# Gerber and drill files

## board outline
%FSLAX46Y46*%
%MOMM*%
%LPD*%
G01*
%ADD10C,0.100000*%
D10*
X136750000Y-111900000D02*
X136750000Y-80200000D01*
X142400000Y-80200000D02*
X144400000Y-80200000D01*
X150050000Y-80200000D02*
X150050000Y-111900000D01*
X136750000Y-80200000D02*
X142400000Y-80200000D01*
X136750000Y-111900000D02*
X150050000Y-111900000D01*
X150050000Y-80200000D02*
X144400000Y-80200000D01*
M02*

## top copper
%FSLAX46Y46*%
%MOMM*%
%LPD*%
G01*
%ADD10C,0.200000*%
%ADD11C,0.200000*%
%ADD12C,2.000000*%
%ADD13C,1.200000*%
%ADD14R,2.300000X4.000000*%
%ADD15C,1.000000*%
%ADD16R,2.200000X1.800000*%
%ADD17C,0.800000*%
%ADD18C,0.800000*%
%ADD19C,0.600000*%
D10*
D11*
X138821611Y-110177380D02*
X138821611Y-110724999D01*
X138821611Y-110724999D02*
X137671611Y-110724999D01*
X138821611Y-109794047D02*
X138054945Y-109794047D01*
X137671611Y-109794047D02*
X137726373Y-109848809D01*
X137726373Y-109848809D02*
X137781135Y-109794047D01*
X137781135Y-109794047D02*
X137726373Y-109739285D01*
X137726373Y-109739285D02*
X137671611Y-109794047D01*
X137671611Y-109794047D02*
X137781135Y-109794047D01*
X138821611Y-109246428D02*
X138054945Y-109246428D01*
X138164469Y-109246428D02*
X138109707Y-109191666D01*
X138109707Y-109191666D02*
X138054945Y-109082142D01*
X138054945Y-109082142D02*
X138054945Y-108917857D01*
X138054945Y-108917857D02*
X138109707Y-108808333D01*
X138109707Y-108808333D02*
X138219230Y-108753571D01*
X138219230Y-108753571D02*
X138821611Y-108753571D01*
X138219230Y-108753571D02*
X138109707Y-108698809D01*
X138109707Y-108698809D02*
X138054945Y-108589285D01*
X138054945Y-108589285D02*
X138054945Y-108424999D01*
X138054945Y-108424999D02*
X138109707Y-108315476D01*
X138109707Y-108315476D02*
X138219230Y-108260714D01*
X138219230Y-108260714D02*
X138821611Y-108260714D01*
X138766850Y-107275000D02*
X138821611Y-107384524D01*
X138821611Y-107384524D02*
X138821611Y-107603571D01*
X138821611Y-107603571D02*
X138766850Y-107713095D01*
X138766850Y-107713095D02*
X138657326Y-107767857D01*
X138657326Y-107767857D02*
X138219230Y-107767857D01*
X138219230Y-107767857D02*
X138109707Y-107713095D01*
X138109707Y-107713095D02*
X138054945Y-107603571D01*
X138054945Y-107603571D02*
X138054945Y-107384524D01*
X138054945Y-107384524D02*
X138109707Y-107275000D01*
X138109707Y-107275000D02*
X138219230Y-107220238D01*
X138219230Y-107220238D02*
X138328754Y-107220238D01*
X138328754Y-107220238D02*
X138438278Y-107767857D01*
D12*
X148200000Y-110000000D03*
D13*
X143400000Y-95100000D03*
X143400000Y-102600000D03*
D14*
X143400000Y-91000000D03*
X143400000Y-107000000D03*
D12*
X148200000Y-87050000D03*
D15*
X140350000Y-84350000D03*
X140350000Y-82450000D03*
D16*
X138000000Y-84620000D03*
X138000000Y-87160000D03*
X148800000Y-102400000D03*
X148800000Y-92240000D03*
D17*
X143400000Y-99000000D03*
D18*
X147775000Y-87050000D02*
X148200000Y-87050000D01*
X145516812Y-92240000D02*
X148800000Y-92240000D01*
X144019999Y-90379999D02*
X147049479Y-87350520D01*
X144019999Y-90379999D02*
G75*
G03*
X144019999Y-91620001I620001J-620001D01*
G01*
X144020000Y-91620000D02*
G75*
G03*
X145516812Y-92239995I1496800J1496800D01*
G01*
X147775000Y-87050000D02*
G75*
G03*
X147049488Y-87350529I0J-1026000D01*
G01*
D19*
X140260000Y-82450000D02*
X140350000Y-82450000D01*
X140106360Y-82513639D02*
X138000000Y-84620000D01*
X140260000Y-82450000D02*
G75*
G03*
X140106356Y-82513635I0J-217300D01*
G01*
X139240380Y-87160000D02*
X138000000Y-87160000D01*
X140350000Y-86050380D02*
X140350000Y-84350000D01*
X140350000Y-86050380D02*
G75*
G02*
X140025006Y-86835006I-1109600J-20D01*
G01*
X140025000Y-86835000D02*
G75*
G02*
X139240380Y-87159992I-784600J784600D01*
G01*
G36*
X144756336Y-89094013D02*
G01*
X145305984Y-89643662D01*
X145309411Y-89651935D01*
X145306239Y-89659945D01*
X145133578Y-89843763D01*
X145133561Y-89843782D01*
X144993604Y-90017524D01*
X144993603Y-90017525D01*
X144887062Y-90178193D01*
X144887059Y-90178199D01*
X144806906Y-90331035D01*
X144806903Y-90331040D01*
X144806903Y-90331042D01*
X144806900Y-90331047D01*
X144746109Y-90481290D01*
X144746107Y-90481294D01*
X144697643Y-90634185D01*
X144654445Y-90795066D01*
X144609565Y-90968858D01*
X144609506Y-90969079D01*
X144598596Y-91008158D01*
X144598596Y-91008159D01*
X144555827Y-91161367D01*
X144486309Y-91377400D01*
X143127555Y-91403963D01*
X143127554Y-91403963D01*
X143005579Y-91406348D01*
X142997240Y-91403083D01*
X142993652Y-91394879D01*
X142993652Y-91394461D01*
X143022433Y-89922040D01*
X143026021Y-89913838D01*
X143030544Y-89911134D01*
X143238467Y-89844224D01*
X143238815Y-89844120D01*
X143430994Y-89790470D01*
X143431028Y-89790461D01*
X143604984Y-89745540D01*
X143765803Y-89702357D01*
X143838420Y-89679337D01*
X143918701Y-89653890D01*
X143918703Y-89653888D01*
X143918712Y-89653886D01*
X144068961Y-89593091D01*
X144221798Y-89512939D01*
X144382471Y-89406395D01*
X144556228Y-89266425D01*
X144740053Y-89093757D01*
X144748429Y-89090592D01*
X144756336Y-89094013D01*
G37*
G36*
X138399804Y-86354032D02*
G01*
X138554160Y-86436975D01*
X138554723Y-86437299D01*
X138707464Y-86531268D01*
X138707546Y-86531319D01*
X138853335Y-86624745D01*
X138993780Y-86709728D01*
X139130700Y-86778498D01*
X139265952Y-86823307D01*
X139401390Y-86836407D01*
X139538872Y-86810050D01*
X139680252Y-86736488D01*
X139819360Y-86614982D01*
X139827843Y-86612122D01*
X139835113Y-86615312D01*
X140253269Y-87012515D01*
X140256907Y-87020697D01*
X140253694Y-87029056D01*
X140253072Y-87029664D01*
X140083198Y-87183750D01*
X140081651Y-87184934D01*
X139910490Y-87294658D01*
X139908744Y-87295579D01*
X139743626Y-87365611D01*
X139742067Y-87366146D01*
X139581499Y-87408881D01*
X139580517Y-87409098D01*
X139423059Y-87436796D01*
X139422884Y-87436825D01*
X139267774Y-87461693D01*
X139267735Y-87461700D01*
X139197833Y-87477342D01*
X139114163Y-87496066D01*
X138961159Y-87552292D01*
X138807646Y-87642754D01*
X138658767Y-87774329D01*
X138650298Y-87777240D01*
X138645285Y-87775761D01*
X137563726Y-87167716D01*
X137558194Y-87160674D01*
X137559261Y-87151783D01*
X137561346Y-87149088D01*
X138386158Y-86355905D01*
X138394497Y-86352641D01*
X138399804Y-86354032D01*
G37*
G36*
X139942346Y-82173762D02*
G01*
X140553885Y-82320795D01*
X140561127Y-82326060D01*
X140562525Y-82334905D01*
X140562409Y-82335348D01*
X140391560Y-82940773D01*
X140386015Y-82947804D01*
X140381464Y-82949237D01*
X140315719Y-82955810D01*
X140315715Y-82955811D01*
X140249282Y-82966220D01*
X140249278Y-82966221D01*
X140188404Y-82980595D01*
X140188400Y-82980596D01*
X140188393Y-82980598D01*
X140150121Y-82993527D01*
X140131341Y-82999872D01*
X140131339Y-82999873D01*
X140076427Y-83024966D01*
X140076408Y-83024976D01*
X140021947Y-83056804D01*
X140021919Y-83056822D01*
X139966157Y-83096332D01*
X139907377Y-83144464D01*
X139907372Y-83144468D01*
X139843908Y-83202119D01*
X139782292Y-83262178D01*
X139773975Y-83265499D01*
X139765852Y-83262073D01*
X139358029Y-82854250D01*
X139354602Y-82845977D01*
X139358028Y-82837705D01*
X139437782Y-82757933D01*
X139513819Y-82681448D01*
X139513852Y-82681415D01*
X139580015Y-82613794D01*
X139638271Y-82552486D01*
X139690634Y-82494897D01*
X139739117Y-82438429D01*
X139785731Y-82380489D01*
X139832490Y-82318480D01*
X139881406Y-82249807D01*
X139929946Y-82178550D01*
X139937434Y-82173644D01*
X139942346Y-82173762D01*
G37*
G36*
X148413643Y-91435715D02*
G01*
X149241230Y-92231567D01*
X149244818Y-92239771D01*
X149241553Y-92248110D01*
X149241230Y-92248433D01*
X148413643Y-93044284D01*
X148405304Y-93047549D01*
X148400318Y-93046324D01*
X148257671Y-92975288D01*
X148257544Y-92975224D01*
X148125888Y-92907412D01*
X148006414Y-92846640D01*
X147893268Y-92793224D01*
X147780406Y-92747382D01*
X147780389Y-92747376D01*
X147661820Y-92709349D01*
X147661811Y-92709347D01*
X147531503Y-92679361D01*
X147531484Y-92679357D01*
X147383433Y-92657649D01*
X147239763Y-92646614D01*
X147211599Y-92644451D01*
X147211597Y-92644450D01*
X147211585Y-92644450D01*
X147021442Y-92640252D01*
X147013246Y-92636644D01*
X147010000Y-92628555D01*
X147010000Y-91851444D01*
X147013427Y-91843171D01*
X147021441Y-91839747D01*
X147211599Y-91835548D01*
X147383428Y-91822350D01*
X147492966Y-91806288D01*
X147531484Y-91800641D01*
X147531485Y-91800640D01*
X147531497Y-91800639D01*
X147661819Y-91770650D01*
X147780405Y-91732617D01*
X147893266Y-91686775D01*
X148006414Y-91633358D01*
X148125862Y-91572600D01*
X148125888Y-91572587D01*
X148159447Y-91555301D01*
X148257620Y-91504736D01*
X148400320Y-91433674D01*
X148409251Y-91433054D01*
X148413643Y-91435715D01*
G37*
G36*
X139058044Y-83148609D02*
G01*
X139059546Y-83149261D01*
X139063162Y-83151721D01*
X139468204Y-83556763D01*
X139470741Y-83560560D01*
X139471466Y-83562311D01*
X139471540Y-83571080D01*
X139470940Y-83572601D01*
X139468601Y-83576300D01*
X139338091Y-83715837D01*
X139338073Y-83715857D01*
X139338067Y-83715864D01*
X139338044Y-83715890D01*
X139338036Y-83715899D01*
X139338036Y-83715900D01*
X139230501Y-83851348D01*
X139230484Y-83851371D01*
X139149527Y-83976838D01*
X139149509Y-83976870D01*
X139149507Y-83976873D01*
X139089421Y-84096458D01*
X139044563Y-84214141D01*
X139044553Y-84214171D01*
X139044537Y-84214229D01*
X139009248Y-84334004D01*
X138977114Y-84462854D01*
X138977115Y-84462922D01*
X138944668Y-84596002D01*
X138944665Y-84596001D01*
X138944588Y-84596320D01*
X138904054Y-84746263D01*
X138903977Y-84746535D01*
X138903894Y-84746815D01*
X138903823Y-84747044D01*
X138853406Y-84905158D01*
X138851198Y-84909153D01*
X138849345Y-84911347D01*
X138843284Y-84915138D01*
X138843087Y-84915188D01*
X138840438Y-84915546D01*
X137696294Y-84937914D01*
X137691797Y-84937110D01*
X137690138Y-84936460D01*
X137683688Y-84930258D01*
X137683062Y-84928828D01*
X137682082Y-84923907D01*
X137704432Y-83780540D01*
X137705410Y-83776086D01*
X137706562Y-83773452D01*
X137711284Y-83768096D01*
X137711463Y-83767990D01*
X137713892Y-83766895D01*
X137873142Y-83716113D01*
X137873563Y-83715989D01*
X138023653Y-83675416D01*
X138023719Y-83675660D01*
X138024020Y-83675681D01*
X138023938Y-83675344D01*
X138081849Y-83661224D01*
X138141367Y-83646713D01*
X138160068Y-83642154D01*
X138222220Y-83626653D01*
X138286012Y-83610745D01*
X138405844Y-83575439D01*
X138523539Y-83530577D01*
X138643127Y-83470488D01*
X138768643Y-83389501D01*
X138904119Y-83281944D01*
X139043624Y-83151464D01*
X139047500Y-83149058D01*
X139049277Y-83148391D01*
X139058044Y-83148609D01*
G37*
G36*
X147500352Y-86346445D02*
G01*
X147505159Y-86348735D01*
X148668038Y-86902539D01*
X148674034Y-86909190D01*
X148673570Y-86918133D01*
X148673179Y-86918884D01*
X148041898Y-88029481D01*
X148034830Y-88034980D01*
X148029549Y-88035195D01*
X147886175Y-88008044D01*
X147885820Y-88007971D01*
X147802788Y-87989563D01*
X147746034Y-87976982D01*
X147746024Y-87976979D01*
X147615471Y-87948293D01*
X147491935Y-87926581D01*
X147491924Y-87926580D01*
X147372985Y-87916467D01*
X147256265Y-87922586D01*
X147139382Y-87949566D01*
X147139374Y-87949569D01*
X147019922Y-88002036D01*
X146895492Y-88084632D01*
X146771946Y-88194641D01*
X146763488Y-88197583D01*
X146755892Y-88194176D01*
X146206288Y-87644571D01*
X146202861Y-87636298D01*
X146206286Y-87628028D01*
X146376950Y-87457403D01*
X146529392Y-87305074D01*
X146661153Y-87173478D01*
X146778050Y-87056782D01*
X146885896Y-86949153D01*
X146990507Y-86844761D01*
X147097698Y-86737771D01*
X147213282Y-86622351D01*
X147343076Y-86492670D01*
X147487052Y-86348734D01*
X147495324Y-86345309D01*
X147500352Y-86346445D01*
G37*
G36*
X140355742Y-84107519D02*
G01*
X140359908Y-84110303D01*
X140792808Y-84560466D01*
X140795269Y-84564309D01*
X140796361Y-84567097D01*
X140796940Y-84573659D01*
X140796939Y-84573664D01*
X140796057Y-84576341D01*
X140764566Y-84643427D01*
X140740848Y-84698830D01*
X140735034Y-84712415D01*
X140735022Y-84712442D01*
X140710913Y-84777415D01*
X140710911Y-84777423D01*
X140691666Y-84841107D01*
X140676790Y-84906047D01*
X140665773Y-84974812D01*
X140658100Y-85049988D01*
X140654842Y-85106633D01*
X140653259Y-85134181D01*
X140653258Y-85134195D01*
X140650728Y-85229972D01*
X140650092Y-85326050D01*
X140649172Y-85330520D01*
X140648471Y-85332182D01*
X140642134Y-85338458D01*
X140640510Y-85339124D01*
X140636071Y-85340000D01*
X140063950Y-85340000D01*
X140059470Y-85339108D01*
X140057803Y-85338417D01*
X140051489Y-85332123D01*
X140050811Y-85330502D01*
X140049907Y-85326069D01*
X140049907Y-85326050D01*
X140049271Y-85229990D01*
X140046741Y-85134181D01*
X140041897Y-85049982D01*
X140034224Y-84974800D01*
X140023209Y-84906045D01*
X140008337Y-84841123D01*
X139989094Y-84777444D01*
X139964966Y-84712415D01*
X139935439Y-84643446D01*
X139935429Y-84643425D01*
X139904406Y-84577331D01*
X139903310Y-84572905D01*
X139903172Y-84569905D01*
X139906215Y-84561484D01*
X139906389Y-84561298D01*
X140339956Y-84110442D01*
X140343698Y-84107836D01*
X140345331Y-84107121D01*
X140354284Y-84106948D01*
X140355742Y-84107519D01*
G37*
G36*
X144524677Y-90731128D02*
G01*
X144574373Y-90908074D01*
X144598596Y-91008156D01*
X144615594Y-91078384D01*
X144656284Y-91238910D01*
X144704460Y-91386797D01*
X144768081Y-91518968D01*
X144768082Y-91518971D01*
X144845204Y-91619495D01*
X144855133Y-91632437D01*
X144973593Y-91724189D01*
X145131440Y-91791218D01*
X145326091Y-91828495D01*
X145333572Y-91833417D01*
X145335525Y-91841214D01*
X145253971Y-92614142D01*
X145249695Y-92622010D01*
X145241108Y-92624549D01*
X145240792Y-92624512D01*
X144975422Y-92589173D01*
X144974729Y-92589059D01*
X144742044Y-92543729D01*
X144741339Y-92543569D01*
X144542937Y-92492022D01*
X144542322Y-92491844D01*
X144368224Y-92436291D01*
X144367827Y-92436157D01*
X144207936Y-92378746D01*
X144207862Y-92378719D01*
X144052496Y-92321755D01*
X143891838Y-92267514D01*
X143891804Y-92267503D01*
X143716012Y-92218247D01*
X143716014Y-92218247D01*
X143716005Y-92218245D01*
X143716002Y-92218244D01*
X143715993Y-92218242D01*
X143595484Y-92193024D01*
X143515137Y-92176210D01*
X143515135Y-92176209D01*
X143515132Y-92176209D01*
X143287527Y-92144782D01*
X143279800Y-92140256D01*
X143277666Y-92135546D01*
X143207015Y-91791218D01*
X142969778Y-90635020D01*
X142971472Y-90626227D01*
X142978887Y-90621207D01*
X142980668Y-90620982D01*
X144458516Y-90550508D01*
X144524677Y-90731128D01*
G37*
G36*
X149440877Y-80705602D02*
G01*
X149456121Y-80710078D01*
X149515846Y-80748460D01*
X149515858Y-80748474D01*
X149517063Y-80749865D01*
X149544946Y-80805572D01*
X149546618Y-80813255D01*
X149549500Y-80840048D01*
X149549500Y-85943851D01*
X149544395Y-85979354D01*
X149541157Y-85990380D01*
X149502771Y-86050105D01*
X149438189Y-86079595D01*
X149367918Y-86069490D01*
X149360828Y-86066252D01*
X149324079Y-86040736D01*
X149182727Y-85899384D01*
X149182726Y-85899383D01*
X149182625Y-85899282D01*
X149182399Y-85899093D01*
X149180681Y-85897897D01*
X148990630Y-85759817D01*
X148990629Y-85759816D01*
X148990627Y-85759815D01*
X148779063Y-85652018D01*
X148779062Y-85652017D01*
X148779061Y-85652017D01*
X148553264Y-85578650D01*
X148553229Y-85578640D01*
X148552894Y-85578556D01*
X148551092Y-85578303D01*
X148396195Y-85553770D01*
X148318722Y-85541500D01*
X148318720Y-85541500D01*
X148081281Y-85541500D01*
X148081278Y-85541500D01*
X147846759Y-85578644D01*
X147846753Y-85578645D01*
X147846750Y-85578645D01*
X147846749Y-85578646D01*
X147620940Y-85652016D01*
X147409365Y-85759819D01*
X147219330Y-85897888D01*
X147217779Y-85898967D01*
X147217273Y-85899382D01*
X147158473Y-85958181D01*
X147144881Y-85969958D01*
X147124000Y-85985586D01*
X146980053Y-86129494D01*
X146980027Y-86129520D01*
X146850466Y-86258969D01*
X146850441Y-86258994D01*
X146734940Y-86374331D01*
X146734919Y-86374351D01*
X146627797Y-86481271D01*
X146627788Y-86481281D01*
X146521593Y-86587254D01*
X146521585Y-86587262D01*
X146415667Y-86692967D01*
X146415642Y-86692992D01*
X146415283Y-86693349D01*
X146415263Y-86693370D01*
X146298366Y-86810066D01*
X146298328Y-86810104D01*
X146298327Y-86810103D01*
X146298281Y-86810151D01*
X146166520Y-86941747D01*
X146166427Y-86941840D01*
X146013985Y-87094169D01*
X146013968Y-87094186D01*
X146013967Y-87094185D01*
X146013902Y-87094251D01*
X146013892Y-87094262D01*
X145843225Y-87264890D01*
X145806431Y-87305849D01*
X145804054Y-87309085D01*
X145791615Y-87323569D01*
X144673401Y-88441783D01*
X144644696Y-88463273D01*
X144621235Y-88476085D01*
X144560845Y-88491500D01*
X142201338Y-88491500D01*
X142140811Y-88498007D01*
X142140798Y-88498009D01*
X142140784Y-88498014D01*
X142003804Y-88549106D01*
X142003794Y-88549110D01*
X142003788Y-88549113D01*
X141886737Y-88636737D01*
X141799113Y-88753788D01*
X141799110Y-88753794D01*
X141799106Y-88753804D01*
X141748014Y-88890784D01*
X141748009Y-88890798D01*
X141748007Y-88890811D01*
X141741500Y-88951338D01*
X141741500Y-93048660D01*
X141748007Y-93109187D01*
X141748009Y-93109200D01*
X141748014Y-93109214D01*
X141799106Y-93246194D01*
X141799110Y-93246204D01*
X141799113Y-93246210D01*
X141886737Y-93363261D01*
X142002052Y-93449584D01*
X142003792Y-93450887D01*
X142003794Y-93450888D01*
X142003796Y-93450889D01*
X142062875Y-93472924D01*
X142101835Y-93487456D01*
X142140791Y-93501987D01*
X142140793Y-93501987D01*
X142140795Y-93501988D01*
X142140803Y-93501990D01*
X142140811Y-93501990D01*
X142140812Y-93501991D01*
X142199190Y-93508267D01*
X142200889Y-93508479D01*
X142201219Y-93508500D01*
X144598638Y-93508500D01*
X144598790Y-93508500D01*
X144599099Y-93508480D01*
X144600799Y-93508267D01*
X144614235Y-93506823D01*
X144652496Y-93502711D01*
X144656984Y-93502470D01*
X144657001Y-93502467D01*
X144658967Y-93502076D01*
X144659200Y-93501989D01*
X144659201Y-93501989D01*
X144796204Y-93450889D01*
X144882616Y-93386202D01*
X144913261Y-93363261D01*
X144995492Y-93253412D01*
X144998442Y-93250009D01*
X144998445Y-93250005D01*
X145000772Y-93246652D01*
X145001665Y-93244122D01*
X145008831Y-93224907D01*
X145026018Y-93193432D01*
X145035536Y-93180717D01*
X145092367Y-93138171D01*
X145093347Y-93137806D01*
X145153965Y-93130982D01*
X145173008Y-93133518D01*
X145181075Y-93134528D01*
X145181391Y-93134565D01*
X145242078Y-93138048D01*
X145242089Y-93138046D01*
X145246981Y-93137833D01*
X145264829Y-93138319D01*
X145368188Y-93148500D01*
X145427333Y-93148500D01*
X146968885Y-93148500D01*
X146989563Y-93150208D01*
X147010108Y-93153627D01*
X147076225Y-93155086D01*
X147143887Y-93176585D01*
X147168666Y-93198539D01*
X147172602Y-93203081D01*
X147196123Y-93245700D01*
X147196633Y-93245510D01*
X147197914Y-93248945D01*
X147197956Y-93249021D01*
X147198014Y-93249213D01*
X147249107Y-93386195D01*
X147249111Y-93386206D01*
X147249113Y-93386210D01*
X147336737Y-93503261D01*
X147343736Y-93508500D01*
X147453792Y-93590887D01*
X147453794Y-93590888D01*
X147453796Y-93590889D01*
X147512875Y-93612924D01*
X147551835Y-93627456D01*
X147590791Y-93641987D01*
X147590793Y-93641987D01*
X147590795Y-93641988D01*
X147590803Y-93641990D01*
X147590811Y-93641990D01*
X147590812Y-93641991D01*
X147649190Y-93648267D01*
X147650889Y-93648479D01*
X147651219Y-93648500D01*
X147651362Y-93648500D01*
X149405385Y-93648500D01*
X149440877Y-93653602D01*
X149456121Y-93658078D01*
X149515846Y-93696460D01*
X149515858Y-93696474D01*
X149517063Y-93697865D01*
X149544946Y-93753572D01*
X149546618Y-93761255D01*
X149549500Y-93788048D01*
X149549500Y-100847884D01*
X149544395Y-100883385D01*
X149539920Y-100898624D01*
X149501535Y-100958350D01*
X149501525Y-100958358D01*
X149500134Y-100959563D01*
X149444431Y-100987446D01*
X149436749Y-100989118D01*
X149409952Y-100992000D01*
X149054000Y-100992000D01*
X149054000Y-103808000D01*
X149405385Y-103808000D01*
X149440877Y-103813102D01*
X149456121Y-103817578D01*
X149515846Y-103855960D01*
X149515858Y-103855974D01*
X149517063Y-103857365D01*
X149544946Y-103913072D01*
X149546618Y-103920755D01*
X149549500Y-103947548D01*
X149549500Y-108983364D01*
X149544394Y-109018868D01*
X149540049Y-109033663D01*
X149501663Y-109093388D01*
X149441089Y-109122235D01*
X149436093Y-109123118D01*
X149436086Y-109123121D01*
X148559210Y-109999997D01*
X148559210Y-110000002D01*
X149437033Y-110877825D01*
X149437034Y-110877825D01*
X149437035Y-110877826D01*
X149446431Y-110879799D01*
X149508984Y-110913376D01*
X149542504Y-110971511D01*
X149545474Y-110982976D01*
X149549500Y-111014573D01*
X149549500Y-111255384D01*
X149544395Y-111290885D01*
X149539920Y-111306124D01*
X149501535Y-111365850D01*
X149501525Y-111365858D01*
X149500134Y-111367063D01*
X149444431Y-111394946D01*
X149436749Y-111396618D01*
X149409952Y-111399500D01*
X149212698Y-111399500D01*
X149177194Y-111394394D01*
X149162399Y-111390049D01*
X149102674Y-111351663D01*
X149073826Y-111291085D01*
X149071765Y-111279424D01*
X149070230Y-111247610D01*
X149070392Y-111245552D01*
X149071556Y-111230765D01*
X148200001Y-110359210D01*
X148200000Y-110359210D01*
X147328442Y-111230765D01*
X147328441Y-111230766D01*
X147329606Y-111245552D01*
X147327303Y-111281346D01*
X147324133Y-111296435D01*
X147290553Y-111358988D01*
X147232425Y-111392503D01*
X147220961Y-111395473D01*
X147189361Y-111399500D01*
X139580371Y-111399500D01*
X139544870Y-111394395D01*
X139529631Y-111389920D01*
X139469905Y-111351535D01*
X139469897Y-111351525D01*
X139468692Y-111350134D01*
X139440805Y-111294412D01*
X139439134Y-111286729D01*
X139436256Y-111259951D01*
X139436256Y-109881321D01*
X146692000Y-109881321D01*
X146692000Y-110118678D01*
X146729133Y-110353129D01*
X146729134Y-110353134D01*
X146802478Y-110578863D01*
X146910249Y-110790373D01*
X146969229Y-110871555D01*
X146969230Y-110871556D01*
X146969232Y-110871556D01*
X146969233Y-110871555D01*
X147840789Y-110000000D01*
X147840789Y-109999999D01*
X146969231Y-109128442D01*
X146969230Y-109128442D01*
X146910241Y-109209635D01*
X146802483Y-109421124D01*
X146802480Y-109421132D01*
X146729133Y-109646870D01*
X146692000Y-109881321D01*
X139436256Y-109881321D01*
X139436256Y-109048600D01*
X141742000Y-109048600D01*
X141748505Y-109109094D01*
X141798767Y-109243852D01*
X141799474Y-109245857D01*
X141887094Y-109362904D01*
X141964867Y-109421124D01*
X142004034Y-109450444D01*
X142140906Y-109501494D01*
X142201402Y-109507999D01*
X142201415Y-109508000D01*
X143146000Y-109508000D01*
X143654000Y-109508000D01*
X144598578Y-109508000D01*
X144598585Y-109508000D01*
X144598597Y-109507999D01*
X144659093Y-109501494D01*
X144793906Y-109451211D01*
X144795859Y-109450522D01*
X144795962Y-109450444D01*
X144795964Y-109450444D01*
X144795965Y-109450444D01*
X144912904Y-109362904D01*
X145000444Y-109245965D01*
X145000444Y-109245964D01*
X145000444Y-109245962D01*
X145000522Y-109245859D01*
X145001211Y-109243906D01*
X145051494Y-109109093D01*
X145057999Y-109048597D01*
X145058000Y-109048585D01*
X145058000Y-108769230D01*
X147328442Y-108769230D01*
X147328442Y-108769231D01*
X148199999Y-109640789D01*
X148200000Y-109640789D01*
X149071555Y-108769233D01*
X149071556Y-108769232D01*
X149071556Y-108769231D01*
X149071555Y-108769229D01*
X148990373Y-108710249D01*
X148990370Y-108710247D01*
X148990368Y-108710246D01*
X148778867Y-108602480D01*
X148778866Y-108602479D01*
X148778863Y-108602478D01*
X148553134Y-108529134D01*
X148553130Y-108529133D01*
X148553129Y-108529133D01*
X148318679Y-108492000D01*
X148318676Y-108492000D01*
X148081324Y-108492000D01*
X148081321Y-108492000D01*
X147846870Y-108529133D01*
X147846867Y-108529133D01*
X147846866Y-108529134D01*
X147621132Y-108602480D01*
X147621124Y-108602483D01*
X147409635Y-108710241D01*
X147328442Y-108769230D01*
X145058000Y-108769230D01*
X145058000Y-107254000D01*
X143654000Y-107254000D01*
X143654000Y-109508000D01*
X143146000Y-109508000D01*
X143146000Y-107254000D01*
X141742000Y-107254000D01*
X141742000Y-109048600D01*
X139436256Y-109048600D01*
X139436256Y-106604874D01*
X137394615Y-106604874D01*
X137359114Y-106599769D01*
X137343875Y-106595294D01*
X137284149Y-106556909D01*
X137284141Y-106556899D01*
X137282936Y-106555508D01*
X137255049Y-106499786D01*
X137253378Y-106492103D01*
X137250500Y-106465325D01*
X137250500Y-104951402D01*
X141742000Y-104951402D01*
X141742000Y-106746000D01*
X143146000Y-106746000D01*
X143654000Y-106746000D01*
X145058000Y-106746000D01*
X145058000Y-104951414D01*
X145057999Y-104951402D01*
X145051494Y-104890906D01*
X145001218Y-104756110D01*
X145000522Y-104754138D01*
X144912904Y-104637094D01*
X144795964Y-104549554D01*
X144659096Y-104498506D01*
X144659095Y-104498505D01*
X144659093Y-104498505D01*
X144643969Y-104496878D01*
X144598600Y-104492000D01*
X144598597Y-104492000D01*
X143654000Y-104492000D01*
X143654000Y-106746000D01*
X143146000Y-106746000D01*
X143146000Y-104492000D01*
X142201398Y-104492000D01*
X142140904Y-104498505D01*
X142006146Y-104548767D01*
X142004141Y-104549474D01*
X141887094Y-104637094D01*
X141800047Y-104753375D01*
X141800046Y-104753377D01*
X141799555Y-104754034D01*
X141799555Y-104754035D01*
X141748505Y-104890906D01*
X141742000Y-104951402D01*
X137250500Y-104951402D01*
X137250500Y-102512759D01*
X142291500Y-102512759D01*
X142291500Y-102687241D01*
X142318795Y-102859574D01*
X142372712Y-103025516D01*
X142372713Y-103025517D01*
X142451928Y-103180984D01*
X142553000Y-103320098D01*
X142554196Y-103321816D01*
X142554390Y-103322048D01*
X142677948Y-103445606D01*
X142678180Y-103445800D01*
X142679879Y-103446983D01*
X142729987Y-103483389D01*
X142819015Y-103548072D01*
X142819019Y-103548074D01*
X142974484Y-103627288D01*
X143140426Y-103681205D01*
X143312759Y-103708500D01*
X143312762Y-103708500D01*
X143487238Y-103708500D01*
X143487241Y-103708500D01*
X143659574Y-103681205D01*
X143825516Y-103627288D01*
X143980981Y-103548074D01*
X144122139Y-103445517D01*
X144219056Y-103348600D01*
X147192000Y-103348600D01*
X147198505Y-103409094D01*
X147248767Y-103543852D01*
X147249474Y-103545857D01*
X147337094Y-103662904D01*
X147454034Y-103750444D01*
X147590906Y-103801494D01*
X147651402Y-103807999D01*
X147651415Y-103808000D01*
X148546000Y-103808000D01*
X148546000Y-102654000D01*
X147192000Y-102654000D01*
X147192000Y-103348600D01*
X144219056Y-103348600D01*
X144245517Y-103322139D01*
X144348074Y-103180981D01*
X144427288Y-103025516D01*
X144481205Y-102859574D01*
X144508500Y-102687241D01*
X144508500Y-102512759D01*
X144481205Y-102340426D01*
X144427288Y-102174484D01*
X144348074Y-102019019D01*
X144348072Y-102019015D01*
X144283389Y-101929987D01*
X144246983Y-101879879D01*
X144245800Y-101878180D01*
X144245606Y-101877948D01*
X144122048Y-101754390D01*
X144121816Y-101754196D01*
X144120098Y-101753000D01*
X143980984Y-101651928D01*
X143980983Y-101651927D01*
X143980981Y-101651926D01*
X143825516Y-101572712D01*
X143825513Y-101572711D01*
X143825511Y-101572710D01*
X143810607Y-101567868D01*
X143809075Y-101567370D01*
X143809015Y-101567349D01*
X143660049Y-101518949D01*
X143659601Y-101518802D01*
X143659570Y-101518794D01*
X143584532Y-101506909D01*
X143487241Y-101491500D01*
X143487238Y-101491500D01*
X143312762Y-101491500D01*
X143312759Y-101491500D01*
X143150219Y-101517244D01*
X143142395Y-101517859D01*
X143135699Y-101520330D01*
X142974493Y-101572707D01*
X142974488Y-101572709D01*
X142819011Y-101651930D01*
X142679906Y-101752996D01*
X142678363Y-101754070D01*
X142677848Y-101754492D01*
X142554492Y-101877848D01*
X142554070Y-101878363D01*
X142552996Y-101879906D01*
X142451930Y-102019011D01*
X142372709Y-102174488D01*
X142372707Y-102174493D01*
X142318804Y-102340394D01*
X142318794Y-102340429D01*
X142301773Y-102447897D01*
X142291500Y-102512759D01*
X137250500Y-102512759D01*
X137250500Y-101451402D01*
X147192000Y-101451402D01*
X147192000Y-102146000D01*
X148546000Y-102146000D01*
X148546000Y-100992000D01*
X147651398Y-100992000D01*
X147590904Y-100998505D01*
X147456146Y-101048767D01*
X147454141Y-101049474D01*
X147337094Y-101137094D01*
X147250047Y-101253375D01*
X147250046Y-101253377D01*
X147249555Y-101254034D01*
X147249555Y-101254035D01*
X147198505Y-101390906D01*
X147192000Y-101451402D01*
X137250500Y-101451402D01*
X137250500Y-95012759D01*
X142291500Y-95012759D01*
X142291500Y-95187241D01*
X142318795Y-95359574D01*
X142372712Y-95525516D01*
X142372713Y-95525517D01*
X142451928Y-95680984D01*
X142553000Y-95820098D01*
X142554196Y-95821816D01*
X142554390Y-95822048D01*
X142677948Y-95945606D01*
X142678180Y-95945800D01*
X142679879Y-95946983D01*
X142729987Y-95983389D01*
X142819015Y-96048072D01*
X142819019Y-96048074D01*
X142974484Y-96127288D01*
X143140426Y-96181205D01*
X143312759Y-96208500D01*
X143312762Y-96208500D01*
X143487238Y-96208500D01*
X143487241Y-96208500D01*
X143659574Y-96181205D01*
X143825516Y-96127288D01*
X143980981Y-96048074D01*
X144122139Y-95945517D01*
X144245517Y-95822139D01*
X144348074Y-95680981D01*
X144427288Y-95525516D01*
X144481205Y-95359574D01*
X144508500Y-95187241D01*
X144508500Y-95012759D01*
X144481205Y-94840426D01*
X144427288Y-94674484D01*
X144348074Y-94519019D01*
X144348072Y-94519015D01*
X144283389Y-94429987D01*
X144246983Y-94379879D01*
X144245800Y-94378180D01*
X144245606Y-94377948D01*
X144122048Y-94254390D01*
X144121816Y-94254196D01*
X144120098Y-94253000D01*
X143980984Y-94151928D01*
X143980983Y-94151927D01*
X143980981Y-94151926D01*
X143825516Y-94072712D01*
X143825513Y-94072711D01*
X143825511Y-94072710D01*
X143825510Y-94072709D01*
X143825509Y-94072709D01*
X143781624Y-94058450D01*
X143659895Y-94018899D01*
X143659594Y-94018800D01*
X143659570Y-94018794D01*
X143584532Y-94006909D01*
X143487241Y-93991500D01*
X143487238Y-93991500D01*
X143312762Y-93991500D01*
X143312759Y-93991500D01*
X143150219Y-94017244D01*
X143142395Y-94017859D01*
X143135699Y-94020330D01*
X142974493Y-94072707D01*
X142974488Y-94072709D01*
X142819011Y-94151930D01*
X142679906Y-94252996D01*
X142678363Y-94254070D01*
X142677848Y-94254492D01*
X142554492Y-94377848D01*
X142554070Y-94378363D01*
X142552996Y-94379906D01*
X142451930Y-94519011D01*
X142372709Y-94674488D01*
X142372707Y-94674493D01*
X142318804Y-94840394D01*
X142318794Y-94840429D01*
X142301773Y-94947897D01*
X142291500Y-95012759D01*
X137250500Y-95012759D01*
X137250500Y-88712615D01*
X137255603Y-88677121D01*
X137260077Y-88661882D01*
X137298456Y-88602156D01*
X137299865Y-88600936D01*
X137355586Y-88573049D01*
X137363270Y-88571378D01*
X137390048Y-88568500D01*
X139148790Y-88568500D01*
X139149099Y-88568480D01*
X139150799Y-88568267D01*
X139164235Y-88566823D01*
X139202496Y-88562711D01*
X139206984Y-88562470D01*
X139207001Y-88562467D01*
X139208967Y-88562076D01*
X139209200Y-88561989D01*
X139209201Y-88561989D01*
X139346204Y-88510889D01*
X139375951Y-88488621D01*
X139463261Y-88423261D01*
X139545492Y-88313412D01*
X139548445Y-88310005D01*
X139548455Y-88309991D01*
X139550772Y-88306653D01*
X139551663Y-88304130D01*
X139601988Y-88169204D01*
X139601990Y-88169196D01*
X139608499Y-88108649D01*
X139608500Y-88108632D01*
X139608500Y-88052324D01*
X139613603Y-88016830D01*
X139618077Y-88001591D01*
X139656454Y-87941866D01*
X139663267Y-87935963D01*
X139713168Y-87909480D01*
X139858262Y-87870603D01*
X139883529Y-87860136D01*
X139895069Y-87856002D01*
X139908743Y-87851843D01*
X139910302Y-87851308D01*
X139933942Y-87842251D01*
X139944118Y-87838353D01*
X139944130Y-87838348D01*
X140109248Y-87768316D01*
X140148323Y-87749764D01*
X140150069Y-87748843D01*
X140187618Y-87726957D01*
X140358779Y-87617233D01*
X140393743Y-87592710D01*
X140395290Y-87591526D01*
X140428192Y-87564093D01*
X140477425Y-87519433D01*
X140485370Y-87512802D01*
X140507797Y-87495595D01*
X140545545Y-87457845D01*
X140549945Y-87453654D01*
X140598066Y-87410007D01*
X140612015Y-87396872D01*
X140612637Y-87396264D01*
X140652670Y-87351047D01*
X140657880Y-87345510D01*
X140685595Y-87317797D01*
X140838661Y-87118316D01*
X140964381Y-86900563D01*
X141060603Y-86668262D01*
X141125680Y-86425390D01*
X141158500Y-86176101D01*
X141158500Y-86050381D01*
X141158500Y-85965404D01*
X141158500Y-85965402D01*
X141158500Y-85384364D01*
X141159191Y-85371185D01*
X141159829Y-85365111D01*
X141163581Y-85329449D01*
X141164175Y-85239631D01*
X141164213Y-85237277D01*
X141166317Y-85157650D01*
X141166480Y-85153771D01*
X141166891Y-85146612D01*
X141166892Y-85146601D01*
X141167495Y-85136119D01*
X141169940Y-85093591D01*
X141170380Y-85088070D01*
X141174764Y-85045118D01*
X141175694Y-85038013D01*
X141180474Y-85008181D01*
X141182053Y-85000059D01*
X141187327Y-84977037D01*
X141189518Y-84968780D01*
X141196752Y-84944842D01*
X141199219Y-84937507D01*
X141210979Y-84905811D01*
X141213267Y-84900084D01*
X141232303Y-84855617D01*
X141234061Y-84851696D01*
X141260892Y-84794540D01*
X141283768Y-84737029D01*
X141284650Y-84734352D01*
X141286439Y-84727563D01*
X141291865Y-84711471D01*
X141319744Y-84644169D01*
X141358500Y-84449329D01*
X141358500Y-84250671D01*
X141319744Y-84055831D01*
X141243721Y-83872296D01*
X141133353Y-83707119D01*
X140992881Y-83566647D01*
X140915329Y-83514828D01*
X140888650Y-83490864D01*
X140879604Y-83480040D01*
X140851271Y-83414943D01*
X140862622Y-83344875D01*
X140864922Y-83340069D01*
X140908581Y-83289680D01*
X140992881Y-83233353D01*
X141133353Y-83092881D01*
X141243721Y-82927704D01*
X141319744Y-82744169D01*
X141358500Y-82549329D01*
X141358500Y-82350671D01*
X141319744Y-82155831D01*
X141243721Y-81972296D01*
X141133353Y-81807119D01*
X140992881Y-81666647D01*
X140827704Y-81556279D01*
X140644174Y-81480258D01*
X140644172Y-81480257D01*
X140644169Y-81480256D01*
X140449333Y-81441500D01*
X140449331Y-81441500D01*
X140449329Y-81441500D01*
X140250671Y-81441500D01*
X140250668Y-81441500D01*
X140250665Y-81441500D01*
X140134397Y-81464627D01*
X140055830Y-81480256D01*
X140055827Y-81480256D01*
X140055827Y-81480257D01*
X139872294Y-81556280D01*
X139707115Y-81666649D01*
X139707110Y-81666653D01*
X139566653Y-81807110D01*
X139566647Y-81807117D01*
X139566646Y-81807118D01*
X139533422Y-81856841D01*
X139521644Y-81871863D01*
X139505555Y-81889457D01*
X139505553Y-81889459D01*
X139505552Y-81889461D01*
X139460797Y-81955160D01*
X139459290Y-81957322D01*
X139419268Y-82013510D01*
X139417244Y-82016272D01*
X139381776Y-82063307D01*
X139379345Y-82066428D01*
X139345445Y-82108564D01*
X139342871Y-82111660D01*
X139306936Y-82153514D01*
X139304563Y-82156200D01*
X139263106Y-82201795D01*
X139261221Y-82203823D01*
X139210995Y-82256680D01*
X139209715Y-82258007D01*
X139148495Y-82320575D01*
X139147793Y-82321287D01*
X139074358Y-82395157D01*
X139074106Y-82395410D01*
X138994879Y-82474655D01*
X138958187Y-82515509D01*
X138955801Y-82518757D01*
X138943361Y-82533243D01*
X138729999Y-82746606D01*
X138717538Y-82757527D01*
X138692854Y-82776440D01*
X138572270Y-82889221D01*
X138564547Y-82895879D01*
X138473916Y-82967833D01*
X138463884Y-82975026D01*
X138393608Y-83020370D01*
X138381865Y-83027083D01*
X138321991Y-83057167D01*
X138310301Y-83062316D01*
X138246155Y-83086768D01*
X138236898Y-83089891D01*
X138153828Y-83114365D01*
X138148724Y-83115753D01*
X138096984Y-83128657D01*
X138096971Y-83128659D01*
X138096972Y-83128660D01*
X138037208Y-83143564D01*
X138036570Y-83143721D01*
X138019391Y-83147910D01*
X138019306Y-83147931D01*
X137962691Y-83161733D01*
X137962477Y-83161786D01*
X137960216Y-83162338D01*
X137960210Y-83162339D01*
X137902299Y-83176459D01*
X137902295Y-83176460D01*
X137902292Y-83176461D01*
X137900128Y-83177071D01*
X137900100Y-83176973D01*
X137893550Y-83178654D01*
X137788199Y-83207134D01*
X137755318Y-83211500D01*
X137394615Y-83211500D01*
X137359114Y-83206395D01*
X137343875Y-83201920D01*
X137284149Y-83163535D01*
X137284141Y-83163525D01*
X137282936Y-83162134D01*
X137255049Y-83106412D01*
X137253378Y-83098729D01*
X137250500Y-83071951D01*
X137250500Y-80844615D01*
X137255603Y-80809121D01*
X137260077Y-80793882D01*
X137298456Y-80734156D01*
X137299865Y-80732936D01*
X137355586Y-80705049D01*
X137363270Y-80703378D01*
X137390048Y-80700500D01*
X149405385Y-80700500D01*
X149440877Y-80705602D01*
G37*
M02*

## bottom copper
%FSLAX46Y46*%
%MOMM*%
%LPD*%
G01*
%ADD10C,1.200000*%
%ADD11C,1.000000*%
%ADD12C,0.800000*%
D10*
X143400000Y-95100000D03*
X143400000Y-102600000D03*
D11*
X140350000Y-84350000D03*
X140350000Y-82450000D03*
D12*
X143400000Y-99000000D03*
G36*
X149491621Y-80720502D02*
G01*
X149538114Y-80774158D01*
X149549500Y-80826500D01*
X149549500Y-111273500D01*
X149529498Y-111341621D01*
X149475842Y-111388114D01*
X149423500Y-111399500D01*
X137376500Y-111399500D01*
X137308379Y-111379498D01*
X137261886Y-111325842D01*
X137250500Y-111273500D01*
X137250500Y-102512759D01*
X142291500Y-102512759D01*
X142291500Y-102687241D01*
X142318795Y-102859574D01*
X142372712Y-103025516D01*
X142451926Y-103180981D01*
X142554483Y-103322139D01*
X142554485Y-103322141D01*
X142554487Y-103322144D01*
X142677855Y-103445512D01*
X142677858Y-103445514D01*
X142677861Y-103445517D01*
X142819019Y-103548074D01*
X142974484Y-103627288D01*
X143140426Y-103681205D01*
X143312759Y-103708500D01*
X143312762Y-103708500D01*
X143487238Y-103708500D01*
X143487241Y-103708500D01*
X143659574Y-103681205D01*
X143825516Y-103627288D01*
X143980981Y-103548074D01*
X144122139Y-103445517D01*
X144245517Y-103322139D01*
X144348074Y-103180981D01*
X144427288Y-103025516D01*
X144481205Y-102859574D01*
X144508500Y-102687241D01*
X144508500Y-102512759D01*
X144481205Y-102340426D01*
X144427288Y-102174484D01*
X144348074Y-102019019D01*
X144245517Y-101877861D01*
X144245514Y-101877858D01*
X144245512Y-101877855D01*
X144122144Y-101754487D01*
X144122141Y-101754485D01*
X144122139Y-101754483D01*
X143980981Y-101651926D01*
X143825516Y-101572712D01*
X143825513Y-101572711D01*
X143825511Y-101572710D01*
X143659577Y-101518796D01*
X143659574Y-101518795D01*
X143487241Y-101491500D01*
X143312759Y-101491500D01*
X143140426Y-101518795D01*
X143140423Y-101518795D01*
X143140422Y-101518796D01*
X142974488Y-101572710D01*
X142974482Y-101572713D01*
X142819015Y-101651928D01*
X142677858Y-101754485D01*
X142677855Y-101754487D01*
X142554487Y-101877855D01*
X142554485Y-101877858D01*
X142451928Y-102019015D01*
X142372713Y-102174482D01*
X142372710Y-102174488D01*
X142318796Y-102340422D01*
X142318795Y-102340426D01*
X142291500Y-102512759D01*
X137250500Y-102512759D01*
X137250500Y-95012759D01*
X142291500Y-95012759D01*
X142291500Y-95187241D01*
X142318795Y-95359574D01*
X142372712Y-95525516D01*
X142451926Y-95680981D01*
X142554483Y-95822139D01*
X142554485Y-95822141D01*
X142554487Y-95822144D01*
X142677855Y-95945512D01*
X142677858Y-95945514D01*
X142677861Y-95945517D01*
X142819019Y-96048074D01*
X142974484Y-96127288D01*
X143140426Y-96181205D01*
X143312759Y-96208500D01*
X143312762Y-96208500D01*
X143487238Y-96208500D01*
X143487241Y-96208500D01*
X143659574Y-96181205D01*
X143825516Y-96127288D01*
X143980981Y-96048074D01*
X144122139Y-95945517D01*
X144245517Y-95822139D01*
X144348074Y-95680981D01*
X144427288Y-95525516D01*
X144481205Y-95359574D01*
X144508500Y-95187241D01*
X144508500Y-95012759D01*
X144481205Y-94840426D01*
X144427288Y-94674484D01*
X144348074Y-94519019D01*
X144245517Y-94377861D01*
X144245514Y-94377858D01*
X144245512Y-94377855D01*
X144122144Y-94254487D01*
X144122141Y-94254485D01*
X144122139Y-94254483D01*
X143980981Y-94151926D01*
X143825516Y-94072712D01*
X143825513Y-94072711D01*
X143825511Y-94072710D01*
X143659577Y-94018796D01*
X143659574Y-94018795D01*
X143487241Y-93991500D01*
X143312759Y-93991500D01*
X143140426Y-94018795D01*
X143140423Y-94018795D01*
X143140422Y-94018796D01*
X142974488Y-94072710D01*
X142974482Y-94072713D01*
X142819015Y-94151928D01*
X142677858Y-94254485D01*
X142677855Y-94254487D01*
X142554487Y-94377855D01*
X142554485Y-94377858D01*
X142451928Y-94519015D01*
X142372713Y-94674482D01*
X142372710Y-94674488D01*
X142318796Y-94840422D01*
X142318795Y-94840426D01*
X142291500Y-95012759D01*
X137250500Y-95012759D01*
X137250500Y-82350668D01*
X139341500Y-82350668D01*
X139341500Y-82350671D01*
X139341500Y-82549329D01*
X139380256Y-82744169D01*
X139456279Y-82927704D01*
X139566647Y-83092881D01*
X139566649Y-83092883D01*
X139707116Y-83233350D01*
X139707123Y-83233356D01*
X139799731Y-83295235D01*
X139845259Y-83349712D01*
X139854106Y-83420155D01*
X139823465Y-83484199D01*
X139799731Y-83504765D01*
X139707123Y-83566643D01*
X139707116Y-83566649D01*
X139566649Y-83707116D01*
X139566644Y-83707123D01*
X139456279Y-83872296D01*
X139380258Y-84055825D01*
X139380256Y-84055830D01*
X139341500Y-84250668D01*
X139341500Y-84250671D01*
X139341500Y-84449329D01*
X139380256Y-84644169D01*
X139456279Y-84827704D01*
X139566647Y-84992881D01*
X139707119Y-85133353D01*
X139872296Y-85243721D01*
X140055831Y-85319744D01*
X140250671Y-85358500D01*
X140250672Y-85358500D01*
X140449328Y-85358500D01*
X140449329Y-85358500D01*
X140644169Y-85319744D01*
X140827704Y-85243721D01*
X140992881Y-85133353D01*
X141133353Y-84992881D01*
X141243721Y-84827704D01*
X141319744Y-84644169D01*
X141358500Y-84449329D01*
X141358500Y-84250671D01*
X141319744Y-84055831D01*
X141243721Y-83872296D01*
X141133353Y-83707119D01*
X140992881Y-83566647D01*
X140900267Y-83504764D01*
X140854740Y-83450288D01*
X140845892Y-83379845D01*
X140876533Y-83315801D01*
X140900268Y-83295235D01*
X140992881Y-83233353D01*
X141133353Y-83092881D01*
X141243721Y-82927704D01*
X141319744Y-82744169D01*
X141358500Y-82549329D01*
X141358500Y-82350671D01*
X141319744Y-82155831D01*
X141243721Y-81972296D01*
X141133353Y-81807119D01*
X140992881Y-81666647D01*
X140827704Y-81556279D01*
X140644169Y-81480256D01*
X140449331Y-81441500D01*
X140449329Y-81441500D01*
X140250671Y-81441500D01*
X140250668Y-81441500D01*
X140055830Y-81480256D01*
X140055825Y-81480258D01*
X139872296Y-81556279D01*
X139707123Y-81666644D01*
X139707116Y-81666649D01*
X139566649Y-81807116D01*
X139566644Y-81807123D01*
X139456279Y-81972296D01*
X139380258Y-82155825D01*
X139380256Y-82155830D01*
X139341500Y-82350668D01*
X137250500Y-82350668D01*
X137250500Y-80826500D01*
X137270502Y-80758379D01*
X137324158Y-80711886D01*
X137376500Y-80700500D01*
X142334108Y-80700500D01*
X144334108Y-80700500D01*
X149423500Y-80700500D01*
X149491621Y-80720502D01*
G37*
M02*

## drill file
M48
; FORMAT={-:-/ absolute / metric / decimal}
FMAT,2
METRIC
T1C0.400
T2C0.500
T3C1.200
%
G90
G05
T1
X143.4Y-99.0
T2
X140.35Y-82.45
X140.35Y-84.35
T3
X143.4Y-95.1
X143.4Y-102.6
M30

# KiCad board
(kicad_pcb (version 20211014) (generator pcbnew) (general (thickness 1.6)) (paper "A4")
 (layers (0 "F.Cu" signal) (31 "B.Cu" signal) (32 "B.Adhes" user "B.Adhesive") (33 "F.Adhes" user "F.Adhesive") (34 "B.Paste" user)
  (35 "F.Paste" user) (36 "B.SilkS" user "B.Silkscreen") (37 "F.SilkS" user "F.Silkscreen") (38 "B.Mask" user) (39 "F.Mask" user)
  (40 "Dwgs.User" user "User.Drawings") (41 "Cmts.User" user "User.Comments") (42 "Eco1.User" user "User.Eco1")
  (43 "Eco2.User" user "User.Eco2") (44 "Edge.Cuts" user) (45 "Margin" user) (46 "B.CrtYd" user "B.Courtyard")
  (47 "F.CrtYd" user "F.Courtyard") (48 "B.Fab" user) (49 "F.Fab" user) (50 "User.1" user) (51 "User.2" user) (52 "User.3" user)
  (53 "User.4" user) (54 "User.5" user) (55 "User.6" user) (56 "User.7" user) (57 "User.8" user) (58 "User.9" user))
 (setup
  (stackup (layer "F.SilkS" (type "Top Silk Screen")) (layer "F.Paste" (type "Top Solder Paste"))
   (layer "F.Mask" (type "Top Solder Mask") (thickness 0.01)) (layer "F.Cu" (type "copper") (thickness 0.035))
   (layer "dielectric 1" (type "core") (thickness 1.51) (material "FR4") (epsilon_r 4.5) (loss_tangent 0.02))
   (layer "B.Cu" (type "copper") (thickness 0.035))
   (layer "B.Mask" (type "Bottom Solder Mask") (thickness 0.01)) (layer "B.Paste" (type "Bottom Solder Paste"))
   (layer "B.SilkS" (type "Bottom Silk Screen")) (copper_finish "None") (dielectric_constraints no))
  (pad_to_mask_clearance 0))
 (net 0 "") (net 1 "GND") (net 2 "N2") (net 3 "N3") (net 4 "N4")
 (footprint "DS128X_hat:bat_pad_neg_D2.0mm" (layer "F.Cu") (at 148.2 110 -90)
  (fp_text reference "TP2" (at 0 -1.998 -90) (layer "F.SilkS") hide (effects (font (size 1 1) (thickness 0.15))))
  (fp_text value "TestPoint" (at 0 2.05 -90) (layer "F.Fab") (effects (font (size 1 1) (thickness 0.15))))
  (pad "1" smd circle (at 0 0 270) (size 2 2) (layers "F.Cu" "F.Mask") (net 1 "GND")))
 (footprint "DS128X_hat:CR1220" (layer "F.Cu") (at 143.4 99 180)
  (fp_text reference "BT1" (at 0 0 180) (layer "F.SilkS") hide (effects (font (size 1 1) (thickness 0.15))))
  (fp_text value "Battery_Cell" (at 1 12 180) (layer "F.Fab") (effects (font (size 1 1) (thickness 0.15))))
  (pad "" thru_hole circle (at 0 3.9 180) (size 1.2 1.2) (drill 1.2) (layers *.Cu "F.SilkS"))
  (pad "" thru_hole circle (at 0 -3.6 180) (size 1.2 1.2) (drill 1.2) (layers *.Cu "F.SilkS"))
  (pad "1" smd rect (at 0 8 180) (size 2.3 4) (layers "F.Cu" "F.Paste" "F.Mask") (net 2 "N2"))
  (pad "2" smd rect (at 0 -8 180) (size 2.3 4) (layers "F.Cu" "F.Paste" "F.Mask") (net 1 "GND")))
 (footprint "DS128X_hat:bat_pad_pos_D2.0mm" (layer "F.Cu") (at 148.2 87.05 -90)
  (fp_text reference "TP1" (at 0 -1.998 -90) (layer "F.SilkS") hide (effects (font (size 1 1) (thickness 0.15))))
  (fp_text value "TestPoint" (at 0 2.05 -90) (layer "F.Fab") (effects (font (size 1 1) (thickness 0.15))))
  (pad "1" smd circle (at 0 0 270) (size 2 2) (layers "F.Cu" "F.Mask") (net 2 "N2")))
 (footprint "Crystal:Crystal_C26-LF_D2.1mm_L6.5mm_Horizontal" (layer "F.Cu") (at 140.35 84.35 90)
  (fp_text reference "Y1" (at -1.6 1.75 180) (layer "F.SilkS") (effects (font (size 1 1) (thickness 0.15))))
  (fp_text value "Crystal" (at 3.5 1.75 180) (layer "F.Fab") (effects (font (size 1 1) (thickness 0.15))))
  (pad "1" thru_hole circle (at 0 0 90) (size 1 1) (drill 0.5) (layers *.Cu *.Mask) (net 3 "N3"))
  (pad "2" thru_hole circle (at 1.9 0 90) (size 1 1) (drill 0.5) (layers *.Cu *.Mask) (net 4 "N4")))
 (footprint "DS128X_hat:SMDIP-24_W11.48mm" (layer "F.Cu") (at 143.4 96.05)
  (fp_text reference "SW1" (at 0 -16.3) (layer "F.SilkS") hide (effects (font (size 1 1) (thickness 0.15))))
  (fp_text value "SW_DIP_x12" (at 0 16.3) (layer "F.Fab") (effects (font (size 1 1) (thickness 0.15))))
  (pad "2" smd rect (at -5.4 -11.43) (size 2.2 1.8) (layers "F.Cu" "F.Paste" "F.Mask") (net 4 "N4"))
  (pad "3" smd rect (at -5.4 -8.89) (size 2.2 1.8) (layers "F.Cu" "F.Paste" "F.Mask") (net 3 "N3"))
  (pad "16" smd rect (at 5.4 6.35) (size 2.2 1.8) (layers "F.Cu" "F.Paste" "F.Mask") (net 1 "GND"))
  (pad "20" smd rect (at 5.4 -3.81) (size 2.2 1.8) (layers "F.Cu" "F.Paste" "F.Mask") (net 2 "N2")))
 (gr_line (start 136.75 111.9) (end 136.75 80.2) (layer "Edge.Cuts") (width 0.1))
 (gr_line (start 142.4 80.2) (end 144.4 80.2) (layer "Edge.Cuts") (width 0.1))
 (gr_line (start 150.05 80.2) (end 150.05 111.9) (layer "Edge.Cuts") (width 0.1))
 (gr_line (start 136.75 80.2) (end 142.4 80.2) (layer "Edge.Cuts") (width 0.1))
 (gr_line (start 136.75 111.9) (end 150.05 111.9) (layer "Edge.Cuts") (width 0.1))
 (gr_line (start 150.05 80.2) (end 144.4 80.2) (layer "Edge.Cuts") (width 0.1))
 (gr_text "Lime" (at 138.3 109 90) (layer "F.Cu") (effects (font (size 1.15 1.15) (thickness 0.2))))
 (segment (start 147.775 87.05) (end 148.2 87.05) (width 0.8) (layer "F.Cu") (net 2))
 (segment (start 145.516812 92.24) (end 148.8 92.24) (width 0.8) (layer "F.Cu") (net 2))
 (segment (start 144.019999 90.379999) (end 147.049479 87.35052) (width 0.8) (layer "F.Cu") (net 2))
 (arc (start 144.019999 90.379999) (mid 143.763187 90.999999) (end 144.02 91.62) (width 0.8) (layer "F.Cu") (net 2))
 (arc (start 144.02 91.62) (mid 144.706743 92.078867) (end 145.516812 92.24) (width 0.8) (layer "F.Cu") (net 2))
 (arc (start 147.775 87.05) (mid 147.382351 87.128102) (end 147.049479 87.35052) (width 0.8) (layer "F.Cu") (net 2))
 (segment (start 140.26 82.45) (end 140.35 82.45) (width 0.6) (layer "F.Cu") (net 4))
 (segment (start 140.10636 82.513639) (end 138 84.62) (width 0.6) (layer "F.Cu") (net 4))
 (arc (start 140.26 82.45) (mid 140.17685 82.466539) (end 140.10636 82.513639) (width 0.6) (layer "F.Cu") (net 4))
 (segment (start 139.24038 87.16) (end 138 87.16) (width 0.6) (layer "F.Cu") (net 3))
 (segment (start 140.35 86.05038) (end 140.35 84.35) (width 0.6) (layer "F.Cu") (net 3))
 (arc (start 140.35 86.05038) (mid 140.265535 86.475013) (end 140.025 86.835) (width 0.6) (layer "F.Cu") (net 3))
 (arc (start 140.025 86.835) (mid 139.665013 87.075535) (end 139.24038 87.16) (width 0.6) (layer "F.Cu") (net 3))
 (via (at 143.4 99) (size 0.8) (drill 0.4) (layers "F.Cu" "B.Cu") (free) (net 1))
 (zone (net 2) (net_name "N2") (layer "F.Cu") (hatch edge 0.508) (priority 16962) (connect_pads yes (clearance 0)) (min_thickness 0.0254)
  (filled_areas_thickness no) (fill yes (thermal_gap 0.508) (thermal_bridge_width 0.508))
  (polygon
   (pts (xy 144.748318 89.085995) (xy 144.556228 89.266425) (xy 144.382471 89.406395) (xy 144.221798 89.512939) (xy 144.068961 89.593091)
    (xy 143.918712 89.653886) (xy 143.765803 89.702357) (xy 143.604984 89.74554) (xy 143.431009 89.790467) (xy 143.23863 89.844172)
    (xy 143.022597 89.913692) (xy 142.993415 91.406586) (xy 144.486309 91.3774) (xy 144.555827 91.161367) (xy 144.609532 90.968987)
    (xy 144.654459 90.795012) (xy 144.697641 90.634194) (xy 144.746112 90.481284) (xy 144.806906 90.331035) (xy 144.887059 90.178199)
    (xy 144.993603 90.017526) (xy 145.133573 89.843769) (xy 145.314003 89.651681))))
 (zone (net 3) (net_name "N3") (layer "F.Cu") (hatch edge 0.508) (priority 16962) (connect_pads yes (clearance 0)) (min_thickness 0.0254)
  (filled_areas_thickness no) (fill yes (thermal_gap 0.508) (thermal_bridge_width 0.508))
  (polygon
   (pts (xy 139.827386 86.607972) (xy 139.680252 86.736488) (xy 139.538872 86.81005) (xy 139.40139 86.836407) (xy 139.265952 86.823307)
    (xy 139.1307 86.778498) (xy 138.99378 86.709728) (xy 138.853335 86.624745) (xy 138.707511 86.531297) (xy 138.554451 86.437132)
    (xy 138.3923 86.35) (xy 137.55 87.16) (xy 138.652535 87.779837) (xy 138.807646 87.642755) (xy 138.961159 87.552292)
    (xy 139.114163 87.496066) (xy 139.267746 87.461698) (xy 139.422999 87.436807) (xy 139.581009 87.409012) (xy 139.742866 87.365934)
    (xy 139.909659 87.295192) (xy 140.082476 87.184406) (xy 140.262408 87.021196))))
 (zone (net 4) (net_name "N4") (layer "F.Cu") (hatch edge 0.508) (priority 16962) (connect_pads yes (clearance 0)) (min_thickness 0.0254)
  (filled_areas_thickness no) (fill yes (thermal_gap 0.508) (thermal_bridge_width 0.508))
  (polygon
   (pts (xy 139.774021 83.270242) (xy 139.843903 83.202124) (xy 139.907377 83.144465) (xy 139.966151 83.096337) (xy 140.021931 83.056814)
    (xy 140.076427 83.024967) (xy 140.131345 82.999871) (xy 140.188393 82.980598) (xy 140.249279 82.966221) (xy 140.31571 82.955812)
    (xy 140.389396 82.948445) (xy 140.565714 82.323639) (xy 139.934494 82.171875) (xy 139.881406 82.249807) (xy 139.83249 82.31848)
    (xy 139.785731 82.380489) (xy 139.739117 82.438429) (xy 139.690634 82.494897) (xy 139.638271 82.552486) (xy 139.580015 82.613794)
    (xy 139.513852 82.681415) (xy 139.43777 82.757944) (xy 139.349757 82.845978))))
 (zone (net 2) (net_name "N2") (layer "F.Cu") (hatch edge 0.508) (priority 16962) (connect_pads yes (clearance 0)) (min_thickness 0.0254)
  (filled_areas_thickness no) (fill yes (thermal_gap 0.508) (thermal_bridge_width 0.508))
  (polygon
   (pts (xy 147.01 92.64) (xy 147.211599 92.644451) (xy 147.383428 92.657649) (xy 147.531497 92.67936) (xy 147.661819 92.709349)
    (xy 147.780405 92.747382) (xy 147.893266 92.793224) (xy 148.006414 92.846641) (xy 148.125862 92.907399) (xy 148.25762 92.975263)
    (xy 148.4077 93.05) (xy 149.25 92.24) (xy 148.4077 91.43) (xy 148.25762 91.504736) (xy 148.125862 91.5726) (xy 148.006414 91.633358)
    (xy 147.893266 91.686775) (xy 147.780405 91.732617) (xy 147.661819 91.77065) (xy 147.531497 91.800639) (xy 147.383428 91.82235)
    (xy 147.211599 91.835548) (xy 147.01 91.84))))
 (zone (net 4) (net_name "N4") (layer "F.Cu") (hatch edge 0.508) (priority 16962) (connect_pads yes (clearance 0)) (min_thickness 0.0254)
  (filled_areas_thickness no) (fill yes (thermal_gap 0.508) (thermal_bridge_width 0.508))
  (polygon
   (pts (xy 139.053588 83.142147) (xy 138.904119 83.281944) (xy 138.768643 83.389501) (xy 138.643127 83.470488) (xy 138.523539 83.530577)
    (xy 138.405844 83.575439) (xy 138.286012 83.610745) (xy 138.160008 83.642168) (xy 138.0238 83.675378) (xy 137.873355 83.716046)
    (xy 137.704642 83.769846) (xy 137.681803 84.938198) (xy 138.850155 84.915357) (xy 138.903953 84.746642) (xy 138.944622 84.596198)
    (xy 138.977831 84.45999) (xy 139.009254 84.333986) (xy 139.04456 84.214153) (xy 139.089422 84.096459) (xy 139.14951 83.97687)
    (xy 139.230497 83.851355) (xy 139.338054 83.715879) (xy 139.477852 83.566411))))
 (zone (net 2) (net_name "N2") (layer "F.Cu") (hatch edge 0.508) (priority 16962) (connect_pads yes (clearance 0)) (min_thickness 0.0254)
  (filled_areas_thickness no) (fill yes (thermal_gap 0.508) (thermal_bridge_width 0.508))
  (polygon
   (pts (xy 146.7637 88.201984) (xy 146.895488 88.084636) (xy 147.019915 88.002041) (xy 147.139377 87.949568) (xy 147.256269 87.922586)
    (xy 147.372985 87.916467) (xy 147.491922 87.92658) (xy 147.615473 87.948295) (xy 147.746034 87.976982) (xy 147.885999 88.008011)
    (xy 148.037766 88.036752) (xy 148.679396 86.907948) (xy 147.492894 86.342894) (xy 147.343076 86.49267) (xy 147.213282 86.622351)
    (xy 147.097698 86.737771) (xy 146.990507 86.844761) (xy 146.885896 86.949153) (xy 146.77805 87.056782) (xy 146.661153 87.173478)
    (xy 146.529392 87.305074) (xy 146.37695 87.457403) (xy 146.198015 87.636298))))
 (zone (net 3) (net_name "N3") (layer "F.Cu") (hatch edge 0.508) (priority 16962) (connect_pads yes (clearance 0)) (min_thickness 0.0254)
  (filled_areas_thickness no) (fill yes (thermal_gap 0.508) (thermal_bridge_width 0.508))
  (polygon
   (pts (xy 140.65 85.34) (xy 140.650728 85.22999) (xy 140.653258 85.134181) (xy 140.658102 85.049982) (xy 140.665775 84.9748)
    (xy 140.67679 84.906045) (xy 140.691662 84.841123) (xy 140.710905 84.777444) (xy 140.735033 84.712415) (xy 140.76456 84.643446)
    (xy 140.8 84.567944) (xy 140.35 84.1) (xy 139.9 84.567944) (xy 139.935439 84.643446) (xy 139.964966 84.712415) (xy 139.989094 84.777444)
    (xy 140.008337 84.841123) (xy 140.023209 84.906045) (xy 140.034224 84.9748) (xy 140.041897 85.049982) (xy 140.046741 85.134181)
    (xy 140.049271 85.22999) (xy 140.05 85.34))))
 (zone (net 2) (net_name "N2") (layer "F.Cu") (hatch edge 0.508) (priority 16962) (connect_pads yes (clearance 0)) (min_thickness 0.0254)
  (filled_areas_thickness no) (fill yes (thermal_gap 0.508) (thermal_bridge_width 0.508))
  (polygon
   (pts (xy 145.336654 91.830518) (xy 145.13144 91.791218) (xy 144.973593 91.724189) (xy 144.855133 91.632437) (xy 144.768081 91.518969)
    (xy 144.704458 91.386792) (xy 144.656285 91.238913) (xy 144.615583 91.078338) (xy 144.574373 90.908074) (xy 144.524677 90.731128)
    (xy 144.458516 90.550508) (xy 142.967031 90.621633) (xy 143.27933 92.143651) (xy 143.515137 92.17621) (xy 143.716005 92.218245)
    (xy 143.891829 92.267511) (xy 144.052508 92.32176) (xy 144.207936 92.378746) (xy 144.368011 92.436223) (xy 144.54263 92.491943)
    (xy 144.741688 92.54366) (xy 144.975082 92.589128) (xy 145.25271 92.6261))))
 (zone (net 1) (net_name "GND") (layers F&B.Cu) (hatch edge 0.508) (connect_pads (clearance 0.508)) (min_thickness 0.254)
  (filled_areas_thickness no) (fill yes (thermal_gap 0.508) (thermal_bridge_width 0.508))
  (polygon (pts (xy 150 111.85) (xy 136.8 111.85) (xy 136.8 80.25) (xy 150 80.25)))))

